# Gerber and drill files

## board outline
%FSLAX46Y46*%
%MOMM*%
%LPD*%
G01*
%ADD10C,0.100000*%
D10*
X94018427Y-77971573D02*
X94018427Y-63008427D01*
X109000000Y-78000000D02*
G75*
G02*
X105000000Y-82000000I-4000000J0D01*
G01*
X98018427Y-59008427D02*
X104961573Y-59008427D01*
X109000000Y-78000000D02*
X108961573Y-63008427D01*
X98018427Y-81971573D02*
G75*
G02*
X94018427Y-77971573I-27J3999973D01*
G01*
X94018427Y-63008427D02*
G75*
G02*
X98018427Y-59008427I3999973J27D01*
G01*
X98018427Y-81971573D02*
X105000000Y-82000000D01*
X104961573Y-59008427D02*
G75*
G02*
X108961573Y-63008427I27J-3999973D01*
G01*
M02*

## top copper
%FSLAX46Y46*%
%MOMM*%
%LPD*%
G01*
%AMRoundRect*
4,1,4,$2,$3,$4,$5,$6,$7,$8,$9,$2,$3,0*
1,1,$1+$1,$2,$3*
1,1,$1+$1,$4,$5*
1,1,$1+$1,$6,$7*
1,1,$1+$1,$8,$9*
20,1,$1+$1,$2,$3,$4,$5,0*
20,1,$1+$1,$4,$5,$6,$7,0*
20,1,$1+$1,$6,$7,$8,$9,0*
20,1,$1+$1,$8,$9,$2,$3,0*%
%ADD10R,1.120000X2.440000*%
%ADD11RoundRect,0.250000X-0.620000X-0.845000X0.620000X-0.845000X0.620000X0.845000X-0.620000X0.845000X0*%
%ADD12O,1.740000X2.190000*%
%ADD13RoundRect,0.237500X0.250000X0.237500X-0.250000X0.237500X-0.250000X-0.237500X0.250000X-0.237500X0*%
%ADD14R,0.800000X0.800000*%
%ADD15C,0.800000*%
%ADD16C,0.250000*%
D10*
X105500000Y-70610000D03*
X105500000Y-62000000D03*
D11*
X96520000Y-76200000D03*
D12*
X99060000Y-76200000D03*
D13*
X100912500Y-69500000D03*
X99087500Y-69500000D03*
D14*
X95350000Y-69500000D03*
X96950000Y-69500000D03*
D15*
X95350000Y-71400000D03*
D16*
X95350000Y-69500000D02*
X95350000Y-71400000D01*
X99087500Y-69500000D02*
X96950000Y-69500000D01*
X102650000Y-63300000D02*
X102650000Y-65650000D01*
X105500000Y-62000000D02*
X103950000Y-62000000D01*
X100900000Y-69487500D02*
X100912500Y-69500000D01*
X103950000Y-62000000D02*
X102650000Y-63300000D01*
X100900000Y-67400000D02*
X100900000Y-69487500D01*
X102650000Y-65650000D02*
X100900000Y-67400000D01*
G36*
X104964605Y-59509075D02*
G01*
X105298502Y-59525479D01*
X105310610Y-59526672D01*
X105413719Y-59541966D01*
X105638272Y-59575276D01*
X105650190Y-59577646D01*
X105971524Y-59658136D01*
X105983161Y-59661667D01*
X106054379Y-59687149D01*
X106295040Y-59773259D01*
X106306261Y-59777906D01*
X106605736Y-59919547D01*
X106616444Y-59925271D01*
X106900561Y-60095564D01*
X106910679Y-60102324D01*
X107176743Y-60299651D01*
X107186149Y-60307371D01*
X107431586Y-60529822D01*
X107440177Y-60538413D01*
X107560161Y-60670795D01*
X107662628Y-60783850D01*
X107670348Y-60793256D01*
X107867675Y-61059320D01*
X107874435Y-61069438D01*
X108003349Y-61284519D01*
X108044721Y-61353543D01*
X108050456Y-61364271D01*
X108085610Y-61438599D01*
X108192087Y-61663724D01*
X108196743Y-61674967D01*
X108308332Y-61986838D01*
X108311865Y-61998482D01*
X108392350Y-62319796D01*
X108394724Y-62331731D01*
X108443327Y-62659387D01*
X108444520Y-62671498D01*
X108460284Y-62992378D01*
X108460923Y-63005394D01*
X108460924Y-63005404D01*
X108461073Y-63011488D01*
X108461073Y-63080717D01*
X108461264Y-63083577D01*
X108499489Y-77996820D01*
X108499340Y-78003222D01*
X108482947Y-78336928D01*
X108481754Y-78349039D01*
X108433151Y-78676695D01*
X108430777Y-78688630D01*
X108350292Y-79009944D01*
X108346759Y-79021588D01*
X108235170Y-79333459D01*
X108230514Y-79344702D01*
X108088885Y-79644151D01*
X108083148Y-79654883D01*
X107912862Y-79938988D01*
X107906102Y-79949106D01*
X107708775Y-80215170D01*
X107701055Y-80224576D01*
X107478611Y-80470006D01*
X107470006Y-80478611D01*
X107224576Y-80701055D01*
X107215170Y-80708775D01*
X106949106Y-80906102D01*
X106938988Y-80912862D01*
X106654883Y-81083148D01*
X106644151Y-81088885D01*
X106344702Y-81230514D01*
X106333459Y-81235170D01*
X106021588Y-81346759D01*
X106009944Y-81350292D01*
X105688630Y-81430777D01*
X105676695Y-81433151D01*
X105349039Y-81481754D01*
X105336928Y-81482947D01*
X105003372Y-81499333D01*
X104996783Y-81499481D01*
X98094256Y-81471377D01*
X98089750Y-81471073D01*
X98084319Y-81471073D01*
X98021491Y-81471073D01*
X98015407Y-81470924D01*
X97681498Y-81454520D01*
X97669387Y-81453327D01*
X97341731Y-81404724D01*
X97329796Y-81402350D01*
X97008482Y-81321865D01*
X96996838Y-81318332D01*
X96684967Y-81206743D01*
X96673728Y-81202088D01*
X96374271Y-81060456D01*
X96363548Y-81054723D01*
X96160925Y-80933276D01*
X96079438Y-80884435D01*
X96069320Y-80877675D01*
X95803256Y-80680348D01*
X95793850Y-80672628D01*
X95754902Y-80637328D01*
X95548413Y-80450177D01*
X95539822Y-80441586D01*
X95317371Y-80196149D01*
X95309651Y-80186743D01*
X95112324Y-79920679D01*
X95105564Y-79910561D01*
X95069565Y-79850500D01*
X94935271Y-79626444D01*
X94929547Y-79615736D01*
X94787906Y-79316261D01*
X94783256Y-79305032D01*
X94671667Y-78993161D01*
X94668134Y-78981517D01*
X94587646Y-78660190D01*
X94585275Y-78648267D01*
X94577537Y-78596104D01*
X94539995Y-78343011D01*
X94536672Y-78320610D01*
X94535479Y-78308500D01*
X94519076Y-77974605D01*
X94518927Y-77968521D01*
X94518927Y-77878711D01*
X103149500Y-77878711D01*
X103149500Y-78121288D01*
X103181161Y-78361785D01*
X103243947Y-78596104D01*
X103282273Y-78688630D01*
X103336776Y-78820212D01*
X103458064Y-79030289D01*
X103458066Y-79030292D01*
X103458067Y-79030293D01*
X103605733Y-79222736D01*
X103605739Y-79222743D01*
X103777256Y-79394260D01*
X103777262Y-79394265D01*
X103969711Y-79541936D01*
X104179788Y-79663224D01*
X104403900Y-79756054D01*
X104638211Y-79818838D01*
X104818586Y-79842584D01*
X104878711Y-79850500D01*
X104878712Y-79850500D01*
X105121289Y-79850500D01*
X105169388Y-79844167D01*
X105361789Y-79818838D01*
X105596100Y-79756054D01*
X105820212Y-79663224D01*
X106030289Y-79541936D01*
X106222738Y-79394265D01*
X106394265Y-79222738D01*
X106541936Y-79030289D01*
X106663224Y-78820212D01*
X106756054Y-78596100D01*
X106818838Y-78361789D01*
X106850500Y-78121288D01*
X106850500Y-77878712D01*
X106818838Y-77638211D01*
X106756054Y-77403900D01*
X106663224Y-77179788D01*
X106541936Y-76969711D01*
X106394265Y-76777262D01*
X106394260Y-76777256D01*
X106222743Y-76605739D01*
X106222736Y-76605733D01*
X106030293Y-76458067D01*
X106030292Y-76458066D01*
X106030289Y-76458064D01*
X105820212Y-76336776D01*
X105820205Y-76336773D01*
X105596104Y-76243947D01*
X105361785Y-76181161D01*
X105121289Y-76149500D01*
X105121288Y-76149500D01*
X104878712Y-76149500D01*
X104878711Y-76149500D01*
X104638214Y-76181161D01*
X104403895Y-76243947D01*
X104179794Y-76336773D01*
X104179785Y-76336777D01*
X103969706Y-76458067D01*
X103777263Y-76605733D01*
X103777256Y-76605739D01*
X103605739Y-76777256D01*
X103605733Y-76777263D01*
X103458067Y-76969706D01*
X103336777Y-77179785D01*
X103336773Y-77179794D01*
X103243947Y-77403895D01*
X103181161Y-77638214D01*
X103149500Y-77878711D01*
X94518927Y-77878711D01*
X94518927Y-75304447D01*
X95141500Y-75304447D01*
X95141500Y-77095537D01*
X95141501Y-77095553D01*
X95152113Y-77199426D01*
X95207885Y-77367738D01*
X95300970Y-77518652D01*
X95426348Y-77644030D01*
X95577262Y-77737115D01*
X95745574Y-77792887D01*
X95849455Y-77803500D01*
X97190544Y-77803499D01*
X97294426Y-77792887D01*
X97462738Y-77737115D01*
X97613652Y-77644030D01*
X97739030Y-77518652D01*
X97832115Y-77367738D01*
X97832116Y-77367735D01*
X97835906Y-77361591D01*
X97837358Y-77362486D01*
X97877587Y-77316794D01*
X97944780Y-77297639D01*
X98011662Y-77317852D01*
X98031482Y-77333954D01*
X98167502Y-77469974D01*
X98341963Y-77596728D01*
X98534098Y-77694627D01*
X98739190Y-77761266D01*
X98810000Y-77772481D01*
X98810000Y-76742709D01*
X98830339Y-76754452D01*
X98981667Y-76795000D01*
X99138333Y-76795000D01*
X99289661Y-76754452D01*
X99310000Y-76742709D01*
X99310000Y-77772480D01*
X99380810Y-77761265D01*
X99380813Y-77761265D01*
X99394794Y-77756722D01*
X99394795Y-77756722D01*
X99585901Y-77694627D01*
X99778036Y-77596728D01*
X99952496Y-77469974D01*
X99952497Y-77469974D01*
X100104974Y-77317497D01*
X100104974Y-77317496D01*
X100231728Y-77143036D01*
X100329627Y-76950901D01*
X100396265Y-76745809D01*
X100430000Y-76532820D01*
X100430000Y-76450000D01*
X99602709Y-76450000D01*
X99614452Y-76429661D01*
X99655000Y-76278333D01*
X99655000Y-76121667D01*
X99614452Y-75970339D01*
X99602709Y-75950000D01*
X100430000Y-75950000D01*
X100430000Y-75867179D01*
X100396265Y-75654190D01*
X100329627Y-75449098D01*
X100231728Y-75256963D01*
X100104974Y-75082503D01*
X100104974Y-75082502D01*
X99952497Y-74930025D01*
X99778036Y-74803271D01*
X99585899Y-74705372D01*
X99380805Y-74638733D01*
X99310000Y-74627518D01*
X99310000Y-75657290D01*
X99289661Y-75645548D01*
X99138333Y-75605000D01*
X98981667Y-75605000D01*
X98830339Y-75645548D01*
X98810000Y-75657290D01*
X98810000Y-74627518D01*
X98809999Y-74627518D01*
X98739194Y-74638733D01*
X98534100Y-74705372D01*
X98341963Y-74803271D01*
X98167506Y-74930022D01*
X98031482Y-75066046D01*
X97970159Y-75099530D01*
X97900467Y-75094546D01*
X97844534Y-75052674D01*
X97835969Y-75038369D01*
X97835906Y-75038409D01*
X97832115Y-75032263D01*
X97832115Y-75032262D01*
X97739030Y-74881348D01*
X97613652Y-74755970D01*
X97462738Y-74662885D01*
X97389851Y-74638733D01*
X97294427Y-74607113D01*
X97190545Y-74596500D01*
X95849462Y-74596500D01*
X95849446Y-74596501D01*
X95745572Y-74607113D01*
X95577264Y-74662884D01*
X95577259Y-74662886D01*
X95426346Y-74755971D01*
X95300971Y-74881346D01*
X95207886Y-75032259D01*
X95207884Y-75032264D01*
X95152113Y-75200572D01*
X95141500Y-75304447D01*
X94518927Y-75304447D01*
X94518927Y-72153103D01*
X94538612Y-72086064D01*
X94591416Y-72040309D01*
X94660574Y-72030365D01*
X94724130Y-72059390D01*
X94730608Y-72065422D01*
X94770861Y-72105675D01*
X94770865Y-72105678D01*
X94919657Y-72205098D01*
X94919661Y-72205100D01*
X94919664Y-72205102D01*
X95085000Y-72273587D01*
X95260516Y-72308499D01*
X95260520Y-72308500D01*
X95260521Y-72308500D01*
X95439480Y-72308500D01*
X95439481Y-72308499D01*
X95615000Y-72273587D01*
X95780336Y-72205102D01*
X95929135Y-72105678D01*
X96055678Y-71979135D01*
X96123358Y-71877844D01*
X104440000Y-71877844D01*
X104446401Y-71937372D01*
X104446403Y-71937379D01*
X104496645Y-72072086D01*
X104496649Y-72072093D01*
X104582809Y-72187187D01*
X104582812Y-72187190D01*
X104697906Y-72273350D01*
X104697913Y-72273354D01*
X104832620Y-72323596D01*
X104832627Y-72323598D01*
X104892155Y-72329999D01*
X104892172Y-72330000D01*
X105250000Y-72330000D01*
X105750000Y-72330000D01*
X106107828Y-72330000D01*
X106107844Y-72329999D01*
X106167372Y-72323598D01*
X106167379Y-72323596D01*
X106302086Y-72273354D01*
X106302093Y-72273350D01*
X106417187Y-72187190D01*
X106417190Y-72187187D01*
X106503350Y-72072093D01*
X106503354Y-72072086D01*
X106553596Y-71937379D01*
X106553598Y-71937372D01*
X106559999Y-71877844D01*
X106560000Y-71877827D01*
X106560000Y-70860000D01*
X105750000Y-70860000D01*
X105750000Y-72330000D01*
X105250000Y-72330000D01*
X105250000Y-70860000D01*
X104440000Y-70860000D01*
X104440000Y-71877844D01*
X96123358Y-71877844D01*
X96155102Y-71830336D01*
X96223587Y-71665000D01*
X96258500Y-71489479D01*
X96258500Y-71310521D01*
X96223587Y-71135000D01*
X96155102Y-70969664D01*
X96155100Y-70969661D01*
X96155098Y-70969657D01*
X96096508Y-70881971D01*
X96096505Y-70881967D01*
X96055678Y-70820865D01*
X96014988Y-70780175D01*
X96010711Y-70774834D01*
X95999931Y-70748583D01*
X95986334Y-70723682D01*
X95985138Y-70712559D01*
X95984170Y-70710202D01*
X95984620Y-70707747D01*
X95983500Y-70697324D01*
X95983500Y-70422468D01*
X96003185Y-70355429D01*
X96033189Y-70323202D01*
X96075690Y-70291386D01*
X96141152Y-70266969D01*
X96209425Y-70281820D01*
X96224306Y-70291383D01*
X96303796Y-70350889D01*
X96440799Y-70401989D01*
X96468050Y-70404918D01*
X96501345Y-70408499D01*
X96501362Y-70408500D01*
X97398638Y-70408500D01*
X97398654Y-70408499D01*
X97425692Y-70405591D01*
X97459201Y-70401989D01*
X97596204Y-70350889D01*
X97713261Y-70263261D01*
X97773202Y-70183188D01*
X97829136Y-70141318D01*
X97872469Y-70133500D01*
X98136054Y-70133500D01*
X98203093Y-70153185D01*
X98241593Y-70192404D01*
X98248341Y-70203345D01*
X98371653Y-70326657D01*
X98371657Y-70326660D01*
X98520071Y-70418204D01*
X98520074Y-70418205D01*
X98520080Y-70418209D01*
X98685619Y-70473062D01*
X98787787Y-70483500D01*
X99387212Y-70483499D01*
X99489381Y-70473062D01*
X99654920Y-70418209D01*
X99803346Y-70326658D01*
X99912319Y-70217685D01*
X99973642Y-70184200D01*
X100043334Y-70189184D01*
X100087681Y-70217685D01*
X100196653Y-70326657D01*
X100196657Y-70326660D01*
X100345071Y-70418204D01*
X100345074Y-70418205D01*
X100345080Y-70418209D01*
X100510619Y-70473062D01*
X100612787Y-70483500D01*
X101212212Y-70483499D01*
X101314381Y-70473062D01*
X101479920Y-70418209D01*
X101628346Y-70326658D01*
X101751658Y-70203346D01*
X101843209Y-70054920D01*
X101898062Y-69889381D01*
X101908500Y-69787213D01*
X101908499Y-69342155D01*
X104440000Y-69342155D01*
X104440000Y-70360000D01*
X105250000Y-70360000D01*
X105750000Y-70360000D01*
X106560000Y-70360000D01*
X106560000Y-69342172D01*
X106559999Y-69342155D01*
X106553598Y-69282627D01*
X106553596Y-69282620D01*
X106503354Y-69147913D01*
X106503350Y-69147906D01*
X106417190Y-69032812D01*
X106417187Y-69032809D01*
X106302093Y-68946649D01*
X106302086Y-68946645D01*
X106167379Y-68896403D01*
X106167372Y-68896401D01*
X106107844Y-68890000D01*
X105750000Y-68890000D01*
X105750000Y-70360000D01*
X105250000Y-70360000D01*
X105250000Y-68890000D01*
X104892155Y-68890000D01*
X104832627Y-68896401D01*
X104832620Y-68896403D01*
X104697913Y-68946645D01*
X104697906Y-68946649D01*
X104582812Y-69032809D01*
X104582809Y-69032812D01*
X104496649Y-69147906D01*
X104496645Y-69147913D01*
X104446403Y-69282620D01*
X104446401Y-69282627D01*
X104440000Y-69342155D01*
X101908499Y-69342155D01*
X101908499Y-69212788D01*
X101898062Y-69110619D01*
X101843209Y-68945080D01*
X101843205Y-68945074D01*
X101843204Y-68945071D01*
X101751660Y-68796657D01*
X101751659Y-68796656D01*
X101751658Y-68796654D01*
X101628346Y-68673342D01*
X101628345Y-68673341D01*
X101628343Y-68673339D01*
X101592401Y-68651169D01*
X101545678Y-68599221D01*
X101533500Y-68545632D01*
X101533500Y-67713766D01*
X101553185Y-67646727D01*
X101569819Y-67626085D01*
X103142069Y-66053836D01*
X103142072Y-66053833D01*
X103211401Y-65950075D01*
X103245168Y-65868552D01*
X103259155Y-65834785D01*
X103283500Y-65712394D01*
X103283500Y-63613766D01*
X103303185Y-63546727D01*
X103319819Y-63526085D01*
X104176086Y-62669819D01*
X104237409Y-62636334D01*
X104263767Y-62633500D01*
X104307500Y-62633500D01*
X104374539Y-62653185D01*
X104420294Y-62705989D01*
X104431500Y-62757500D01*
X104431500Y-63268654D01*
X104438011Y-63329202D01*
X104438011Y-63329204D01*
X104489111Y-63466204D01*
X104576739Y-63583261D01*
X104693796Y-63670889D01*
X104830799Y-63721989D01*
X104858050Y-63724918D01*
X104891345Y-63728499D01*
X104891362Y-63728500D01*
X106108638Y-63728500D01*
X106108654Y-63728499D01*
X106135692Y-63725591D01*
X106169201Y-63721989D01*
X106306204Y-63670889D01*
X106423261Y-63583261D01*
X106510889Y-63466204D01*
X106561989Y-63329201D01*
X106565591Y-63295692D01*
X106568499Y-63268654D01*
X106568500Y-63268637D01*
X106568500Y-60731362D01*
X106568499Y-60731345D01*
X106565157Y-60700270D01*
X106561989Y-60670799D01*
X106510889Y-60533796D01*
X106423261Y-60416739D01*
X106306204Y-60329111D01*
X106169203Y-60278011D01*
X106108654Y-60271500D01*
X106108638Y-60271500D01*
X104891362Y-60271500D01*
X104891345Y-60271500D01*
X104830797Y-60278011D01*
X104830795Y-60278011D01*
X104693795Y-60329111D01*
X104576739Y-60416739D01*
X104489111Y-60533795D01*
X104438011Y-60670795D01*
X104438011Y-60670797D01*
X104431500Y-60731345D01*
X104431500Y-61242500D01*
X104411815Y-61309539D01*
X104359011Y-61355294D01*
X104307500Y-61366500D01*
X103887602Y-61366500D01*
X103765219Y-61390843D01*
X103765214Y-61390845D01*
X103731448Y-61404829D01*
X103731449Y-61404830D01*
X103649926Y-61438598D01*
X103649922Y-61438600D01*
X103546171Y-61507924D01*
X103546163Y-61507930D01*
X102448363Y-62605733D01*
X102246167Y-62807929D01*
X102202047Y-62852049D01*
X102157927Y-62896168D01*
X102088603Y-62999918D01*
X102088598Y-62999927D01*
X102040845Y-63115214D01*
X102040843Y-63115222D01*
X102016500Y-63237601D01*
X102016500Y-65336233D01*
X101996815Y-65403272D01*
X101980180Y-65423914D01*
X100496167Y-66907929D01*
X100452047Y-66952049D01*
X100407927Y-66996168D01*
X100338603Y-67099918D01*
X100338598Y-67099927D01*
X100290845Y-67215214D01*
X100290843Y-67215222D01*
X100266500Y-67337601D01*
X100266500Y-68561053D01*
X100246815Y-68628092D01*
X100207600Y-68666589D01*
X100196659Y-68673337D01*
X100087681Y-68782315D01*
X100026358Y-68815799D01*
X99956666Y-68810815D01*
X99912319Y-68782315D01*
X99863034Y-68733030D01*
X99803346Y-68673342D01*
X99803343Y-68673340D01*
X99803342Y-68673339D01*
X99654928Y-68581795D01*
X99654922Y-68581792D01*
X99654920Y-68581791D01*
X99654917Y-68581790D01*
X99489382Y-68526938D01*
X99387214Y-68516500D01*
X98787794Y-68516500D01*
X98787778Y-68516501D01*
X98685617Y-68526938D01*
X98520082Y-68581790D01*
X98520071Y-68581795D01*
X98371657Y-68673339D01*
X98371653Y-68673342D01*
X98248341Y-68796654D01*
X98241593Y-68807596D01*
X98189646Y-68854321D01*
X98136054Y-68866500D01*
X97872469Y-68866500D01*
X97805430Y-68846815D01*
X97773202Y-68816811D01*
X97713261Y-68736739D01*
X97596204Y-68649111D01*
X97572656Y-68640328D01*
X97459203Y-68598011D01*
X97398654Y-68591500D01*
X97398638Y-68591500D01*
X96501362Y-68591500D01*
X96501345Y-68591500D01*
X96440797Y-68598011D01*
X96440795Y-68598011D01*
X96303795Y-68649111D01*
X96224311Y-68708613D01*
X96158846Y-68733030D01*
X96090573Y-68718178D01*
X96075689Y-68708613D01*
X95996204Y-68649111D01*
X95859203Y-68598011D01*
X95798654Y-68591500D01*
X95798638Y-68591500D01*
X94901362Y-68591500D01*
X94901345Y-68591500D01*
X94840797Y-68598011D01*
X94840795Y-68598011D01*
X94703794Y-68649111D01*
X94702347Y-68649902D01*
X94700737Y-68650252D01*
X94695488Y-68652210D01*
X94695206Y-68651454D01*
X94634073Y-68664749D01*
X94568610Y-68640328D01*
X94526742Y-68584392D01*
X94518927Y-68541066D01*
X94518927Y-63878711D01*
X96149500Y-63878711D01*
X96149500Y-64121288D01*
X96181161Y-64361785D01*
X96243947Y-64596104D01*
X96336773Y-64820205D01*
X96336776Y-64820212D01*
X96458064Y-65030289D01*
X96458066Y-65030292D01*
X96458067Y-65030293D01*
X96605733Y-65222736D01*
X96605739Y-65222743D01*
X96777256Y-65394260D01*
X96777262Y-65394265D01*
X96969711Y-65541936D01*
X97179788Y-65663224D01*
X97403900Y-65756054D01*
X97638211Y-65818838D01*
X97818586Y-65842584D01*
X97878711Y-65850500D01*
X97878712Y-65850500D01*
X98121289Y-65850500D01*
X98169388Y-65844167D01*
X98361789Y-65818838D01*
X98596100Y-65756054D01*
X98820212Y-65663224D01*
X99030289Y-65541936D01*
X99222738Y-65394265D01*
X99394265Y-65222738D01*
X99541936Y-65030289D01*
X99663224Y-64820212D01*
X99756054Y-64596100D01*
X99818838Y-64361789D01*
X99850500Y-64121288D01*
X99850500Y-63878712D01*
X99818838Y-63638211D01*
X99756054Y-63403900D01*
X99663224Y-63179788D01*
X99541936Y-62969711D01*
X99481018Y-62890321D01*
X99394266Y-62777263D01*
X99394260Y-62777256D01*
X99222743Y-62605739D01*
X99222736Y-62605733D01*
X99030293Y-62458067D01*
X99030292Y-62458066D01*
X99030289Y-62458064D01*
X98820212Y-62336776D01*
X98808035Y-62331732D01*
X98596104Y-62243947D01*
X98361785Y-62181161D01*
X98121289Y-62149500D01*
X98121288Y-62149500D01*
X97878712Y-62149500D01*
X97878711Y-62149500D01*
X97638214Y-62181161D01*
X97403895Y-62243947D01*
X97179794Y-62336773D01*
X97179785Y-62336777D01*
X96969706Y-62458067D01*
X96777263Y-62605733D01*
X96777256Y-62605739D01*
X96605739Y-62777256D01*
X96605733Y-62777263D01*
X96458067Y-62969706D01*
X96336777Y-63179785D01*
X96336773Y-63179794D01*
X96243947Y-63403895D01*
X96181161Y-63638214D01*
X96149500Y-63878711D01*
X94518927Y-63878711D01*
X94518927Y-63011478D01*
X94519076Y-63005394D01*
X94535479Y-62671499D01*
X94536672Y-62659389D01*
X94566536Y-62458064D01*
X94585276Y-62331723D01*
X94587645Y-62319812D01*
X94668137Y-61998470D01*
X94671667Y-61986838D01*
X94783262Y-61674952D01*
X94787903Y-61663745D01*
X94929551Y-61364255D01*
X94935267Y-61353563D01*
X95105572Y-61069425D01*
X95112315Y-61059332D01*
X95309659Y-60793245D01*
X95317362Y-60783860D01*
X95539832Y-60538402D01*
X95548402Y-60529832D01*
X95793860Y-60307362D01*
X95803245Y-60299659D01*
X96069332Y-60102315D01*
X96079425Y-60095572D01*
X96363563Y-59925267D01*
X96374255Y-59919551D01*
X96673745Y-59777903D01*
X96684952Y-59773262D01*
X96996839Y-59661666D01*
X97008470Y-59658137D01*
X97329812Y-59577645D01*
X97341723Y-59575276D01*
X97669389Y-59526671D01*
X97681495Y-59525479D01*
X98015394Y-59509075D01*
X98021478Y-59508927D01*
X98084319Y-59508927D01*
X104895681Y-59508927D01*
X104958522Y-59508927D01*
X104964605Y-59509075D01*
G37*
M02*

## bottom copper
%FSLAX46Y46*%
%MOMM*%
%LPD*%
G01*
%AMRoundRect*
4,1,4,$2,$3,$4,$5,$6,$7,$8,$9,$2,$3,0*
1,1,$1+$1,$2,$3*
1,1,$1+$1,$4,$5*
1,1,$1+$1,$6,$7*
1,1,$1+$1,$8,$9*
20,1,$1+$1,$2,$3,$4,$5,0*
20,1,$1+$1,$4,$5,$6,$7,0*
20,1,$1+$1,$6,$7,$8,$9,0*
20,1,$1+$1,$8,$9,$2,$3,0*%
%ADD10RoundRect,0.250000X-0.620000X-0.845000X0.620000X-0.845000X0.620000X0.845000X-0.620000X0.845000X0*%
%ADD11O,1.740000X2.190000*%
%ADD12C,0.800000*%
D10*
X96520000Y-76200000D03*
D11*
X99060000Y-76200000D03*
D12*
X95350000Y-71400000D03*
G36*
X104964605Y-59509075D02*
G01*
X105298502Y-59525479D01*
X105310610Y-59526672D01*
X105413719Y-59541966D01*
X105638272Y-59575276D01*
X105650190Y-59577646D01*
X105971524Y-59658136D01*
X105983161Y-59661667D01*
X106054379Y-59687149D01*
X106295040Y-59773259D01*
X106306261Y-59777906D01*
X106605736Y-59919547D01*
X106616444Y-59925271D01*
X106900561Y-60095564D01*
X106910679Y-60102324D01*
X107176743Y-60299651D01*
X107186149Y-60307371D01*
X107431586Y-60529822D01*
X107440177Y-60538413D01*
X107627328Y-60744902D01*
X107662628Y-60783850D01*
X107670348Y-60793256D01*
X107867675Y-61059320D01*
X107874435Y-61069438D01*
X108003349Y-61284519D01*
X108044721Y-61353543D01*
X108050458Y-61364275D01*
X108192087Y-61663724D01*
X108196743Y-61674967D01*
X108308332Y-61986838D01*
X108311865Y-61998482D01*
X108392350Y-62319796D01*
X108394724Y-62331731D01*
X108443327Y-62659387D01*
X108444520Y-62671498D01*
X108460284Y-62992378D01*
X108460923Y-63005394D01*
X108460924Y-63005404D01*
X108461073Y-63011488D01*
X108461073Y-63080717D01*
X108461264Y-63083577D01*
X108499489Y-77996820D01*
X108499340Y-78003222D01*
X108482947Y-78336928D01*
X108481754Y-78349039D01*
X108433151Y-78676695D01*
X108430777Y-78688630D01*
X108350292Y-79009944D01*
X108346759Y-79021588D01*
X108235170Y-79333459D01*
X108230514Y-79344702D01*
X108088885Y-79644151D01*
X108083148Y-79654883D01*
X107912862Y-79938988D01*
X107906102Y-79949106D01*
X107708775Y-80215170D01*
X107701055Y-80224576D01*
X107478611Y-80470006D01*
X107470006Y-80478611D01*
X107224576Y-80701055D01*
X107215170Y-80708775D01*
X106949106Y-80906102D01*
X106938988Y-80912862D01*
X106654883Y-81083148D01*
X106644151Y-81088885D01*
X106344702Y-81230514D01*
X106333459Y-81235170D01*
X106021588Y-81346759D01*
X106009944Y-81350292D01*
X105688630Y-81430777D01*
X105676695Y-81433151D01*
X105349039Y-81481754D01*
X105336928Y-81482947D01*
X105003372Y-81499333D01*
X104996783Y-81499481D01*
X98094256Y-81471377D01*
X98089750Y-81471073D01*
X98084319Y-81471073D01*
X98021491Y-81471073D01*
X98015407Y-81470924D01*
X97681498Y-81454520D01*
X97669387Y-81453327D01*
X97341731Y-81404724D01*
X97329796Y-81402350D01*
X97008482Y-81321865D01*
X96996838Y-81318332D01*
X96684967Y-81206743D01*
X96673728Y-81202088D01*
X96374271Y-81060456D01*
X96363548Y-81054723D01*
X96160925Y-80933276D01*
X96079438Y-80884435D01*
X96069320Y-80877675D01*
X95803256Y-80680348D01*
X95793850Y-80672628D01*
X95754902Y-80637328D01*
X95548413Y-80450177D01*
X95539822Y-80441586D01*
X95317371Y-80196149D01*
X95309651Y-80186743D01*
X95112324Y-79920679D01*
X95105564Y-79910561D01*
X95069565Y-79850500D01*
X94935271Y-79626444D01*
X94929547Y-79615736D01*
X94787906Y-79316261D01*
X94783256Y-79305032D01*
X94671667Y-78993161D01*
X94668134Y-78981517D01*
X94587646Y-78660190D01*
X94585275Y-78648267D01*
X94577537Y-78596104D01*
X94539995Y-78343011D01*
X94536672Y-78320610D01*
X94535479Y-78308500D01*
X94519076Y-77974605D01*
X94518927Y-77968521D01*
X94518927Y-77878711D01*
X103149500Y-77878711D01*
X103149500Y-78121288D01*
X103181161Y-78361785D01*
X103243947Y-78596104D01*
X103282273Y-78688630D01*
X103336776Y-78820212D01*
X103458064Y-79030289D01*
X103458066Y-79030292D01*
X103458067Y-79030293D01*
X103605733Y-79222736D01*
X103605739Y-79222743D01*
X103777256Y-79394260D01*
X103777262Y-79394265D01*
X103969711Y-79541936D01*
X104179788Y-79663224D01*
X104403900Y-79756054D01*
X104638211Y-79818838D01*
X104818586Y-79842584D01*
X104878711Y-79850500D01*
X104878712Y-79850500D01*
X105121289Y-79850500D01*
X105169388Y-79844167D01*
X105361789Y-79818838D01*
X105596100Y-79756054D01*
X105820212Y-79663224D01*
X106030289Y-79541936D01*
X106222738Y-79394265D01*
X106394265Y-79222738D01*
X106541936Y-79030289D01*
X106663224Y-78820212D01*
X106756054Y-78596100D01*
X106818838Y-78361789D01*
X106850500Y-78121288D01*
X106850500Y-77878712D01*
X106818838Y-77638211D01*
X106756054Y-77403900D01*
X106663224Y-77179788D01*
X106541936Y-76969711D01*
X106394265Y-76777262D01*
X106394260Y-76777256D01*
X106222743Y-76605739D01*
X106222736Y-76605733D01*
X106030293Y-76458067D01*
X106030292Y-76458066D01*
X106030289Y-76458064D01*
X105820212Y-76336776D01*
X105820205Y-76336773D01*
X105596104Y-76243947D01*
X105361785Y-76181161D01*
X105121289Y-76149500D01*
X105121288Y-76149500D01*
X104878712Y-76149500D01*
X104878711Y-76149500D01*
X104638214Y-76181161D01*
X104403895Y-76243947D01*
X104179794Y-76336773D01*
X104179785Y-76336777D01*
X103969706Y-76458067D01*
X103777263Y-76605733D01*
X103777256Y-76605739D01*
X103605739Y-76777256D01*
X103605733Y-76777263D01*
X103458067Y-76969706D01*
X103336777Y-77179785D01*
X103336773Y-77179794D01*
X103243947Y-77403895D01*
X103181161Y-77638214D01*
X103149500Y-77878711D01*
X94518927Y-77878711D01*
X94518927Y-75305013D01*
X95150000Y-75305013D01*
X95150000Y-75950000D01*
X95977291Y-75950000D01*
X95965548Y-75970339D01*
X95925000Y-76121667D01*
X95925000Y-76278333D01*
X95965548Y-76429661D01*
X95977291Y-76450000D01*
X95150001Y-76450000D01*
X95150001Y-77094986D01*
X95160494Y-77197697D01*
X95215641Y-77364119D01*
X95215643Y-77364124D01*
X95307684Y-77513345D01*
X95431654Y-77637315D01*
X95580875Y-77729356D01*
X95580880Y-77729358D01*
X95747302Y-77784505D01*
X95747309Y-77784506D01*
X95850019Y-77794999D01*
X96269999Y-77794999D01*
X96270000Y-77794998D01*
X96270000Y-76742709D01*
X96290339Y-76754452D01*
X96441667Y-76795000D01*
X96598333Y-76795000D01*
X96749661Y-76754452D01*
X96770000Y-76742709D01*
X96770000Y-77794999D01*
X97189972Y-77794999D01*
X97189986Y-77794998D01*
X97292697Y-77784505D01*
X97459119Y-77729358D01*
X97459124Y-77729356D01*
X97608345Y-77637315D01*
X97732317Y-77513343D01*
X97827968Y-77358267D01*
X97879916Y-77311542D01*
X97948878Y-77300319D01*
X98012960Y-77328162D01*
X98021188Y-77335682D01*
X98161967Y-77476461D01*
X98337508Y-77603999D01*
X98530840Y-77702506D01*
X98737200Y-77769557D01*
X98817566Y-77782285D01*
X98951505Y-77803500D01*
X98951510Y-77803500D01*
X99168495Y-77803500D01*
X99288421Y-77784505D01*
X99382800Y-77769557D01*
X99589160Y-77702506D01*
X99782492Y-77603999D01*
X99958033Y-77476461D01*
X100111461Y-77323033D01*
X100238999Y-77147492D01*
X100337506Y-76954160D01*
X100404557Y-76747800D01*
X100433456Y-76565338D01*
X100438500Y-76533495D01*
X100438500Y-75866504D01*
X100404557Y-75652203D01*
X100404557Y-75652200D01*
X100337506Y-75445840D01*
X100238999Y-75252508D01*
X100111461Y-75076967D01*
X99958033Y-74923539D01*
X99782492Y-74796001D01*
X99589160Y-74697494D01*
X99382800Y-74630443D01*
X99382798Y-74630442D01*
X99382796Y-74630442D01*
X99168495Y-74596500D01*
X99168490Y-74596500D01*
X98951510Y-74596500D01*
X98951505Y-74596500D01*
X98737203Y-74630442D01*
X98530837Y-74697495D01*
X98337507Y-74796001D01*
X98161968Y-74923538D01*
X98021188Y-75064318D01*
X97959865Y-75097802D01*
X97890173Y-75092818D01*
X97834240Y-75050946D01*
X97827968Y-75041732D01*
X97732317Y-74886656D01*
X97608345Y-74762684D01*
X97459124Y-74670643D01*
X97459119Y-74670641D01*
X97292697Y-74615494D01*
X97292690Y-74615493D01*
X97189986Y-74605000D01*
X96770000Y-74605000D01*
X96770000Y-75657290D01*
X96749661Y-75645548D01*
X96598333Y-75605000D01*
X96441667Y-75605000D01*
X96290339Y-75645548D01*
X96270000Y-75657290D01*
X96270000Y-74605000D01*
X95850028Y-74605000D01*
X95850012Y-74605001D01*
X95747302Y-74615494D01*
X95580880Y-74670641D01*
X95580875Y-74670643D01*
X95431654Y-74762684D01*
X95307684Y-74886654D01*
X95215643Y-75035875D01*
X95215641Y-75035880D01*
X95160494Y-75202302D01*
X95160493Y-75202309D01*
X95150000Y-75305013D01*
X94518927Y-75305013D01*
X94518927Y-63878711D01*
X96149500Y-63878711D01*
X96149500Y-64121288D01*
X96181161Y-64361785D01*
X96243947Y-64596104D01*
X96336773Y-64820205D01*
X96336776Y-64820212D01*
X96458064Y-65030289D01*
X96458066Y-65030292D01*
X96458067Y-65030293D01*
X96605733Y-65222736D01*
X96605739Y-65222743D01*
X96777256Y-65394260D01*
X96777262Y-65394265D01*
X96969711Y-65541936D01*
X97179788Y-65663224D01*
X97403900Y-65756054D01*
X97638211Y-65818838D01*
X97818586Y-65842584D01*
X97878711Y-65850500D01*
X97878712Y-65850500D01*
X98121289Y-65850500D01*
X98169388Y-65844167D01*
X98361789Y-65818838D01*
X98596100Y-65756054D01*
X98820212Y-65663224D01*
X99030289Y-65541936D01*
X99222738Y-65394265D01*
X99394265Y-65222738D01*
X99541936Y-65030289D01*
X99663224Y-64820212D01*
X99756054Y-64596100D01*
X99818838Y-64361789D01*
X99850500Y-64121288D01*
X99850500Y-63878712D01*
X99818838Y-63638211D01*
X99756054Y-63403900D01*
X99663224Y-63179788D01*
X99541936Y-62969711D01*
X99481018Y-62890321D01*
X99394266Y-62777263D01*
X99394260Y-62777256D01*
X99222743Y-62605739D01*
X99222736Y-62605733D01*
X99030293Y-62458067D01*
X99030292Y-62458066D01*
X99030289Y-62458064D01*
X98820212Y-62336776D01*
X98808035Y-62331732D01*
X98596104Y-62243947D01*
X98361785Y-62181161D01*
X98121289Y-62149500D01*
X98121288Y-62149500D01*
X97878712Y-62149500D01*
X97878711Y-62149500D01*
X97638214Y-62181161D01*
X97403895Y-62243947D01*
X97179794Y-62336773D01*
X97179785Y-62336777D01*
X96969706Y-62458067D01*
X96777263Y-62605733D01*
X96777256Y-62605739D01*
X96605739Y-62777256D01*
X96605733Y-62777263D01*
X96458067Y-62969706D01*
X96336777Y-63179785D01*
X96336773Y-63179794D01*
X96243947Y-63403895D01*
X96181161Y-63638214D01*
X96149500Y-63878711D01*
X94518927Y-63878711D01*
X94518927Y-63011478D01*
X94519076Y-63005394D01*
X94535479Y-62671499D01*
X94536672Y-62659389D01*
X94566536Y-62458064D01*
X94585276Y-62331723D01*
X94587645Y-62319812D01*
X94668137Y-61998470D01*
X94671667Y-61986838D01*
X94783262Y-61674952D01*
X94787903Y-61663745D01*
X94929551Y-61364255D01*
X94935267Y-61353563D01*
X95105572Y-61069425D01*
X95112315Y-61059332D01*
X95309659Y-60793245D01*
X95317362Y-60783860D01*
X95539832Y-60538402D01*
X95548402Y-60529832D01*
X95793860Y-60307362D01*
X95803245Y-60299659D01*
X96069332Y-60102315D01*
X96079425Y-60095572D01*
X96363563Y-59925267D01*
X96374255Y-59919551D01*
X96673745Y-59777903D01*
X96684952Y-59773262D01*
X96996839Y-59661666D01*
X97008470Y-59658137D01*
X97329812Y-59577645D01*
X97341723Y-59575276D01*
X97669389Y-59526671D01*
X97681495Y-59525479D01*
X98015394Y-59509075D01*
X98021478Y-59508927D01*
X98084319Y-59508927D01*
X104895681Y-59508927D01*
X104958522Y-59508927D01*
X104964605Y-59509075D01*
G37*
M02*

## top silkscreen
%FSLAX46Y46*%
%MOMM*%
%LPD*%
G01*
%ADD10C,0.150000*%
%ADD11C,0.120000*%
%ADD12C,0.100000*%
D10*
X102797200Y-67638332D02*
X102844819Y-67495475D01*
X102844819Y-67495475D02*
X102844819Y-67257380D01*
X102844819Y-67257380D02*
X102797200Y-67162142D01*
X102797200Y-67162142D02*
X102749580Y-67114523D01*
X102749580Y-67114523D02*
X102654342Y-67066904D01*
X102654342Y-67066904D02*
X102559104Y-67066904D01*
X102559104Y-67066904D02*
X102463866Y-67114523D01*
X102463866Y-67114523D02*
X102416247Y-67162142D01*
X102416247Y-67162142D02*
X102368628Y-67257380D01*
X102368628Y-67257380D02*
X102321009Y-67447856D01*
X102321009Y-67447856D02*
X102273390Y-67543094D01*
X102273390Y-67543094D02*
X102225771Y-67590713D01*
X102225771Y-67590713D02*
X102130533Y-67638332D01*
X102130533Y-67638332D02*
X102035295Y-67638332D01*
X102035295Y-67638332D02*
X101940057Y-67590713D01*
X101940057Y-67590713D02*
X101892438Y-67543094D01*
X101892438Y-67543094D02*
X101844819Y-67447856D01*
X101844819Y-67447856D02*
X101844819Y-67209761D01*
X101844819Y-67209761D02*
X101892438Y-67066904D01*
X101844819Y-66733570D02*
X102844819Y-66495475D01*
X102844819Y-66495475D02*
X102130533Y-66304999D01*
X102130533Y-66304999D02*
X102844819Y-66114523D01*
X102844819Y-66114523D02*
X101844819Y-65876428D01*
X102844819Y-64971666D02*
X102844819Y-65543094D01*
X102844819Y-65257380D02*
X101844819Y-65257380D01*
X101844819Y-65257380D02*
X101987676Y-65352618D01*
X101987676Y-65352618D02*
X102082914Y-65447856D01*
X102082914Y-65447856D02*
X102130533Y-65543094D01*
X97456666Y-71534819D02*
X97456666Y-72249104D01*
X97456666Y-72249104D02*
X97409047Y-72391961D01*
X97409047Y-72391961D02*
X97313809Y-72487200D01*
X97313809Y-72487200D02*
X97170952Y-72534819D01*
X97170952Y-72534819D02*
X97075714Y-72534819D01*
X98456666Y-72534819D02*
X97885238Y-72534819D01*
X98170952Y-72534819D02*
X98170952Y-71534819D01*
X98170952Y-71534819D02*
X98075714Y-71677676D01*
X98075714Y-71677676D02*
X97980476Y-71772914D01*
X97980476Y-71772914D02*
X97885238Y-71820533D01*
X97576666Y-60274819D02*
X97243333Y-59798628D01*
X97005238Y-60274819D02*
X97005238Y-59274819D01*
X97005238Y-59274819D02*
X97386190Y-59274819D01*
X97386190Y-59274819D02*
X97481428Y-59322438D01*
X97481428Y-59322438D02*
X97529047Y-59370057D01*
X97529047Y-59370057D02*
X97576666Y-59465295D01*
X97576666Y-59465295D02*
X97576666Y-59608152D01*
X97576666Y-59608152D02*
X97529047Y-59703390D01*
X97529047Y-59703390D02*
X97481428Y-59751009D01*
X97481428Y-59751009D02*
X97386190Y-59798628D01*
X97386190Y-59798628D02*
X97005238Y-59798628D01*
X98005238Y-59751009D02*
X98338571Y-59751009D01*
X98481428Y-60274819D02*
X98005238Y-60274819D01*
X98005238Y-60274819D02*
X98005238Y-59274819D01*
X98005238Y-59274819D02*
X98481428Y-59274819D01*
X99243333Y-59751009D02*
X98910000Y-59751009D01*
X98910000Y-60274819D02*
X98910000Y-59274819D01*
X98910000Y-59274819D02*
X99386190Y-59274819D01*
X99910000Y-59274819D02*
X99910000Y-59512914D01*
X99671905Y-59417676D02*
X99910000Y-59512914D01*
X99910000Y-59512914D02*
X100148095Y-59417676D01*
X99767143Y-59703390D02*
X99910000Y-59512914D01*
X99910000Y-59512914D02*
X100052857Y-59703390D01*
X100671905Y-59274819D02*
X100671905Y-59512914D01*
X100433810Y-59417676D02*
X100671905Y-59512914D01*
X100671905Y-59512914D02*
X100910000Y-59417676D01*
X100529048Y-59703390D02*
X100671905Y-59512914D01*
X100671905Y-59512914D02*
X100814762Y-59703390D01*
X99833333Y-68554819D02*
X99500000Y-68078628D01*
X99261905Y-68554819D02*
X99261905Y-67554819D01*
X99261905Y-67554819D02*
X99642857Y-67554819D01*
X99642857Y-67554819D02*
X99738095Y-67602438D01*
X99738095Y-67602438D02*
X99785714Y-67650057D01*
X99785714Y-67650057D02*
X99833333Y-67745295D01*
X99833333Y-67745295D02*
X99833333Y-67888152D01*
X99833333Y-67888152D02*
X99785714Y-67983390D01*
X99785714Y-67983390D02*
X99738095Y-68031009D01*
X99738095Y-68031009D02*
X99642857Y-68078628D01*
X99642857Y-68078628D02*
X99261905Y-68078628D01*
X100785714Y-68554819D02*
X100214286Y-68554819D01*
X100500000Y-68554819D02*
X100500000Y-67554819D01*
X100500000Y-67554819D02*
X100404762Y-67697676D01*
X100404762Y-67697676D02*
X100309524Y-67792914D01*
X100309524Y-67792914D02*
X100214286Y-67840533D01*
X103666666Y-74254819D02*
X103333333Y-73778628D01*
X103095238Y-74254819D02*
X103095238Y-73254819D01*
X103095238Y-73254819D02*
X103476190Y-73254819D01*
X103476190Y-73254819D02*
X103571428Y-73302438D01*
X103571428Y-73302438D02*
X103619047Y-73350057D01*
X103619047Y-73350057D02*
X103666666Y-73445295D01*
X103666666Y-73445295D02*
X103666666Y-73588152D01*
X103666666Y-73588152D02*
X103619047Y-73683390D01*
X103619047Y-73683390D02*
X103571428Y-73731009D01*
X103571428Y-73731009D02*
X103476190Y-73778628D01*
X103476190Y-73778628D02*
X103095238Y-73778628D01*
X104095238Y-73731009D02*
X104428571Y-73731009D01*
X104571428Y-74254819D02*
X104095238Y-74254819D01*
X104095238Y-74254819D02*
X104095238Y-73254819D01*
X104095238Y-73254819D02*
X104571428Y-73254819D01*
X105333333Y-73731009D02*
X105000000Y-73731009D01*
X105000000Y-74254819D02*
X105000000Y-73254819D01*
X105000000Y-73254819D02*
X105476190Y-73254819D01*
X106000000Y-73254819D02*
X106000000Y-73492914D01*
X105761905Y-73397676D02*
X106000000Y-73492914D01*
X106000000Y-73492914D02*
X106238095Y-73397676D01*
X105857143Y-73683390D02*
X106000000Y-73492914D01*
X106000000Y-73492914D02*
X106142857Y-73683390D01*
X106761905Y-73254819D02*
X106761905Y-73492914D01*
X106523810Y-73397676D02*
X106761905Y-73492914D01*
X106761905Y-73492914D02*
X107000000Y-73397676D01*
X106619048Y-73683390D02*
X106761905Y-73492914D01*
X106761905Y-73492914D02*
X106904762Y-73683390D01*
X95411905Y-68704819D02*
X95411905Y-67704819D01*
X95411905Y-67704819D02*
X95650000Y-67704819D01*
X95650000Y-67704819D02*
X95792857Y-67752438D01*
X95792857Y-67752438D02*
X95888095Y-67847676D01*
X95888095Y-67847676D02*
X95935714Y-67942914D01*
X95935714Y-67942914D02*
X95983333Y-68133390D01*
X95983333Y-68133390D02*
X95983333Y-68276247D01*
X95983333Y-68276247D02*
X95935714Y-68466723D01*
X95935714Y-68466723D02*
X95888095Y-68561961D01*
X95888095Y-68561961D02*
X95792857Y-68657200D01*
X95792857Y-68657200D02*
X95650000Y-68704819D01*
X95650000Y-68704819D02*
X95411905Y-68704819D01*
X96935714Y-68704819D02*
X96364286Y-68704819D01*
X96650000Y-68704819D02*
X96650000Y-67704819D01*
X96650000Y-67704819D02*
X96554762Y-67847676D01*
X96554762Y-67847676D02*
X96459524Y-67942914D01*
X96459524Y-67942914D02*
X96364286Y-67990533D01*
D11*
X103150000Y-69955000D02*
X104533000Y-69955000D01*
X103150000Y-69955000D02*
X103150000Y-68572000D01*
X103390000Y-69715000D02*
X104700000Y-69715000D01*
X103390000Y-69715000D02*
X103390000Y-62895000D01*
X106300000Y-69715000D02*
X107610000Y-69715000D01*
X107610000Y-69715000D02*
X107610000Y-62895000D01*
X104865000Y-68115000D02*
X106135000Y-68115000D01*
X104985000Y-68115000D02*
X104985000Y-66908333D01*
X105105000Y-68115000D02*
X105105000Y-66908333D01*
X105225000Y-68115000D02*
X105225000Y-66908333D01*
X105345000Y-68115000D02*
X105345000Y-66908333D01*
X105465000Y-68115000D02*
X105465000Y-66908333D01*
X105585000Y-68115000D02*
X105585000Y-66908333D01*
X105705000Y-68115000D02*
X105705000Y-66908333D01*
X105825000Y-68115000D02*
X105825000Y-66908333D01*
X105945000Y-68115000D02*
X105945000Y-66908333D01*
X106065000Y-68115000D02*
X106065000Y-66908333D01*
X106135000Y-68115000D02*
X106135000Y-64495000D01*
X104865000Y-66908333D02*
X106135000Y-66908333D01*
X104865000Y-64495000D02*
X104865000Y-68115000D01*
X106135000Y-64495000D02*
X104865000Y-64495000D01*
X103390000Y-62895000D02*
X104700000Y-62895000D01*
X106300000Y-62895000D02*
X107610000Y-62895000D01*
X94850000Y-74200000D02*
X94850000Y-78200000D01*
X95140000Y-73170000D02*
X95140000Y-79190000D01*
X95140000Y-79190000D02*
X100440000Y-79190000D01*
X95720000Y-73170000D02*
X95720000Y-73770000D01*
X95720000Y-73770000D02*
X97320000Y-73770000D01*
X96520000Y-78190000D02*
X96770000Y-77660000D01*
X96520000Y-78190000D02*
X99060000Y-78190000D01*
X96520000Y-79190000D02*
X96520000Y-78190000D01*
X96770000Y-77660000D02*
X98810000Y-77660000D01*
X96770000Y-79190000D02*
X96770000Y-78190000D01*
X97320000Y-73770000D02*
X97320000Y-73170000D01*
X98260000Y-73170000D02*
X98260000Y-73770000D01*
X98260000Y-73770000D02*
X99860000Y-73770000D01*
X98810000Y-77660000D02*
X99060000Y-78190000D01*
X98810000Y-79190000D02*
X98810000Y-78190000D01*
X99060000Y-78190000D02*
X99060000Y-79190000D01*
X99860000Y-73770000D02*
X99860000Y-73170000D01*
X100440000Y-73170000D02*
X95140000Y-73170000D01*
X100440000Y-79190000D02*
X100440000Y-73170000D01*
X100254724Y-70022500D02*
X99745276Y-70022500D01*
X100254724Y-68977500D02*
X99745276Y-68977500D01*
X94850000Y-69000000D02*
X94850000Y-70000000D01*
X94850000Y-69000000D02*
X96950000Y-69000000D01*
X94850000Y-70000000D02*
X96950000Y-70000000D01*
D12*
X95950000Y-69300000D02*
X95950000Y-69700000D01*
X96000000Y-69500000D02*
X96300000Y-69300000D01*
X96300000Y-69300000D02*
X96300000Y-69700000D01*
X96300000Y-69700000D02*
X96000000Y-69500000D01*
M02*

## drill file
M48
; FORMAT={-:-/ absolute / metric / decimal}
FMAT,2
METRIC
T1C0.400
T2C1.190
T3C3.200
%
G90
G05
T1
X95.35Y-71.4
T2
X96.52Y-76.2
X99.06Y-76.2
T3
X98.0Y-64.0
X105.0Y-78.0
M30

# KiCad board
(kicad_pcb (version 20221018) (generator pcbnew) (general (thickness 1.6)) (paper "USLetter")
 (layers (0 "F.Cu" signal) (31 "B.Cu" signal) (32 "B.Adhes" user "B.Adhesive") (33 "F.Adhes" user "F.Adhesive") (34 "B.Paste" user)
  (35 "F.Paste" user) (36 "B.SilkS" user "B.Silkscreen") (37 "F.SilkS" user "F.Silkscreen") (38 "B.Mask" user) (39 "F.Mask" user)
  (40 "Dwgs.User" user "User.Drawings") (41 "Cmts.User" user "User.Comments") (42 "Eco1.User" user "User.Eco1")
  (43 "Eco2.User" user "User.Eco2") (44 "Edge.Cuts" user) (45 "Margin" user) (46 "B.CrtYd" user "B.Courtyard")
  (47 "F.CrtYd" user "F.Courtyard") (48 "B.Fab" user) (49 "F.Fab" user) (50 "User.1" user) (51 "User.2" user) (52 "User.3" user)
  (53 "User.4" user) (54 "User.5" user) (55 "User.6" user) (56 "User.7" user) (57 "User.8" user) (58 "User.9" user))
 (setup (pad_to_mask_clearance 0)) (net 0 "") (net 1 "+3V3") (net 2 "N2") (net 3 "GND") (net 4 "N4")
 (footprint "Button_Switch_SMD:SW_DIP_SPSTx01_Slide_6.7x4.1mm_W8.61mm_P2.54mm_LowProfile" (layer "F.Cu") (at 105.5 66.305 90)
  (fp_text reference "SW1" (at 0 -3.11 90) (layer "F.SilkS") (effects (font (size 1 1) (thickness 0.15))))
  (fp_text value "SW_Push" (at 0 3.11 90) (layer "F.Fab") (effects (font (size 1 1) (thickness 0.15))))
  (fp_line (start -3.65 -2.35) (end -3.65 -0.967) (stroke (width 0.12) (type solid)) (layer "F.SilkS"))
  (fp_line (start -3.65 -2.35) (end -2.267 -2.35) (stroke (width 0.12) (type solid)) (layer "F.SilkS"))
  (fp_line (start -3.41 -2.11) (end -3.41 -0.8) (stroke (width 0.12) (type solid)) (layer "F.SilkS"))
  (fp_line (start -3.41 -2.11) (end 3.41 -2.11) (stroke (width 0.12) (type solid)) (layer "F.SilkS"))
  (fp_line (start -3.41 0.8) (end -3.41 2.11) (stroke (width 0.12) (type solid)) (layer "F.SilkS"))
  (fp_line (start -3.41 2.11) (end 3.41 2.11) (stroke (width 0.12) (type solid)) (layer "F.SilkS"))
  (fp_line (start -1.81 -0.635) (end -1.81 0.635) (stroke (width 0.12) (type solid)) (layer "F.SilkS"))
  (fp_line (start -1.81 -0.515) (end -0.603333 -0.515) (stroke (width 0.12) (type solid)) (layer "F.SilkS"))
  (fp_line (start -1.81 -0.395) (end -0.603333 -0.395) (stroke (width 0.12) (type solid)) (layer "F.SilkS"))
  (fp_line (start -1.81 -0.275) (end -0.603333 -0.275) (stroke (width 0.12) (type solid)) (layer "F.SilkS"))
  (fp_line (start -1.81 -0.155) (end -0.603333 -0.155) (stroke (width 0.12) (type solid)) (layer "F.SilkS"))
  (fp_line (start -1.81 -0.035) (end -0.603333 -0.035) (stroke (width 0.12) (type solid)) (layer "F.SilkS"))
  (fp_line (start -1.81 0.085) (end -0.603333 0.085) (stroke (width 0.12) (type solid)) (layer "F.SilkS"))
  (fp_line (start -1.81 0.205) (end -0.603333 0.205) (stroke (width 0.12) (type solid)) (layer "F.SilkS"))
  (fp_line (start -1.81 0.325) (end -0.603333 0.325) (stroke (width 0.12) (type solid)) (layer "F.SilkS"))
  (fp_line (start -1.81 0.445) (end -0.603333 0.445) (stroke (width 0.12) (type solid)) (layer "F.SilkS"))
  (fp_line (start -1.81 0.565) (end -0.603333 0.565) (stroke (width 0.12) (type solid)) (layer "F.SilkS"))
  (fp_line (start -1.81 0.635) (end 1.81 0.635) (stroke (width 0.12) (type solid)) (layer "F.SilkS"))
  (fp_line (start -0.603333 -0.635) (end -0.603333 0.635) (stroke (width 0.12) (type solid)) (layer "F.SilkS"))
  (fp_line (start 1.81 -0.635) (end -1.81 -0.635) (stroke (width 0.12) (type solid)) (layer "F.SilkS"))
  (fp_line (start 1.81 0.635) (end 1.81 -0.635) (stroke (width 0.12) (type solid)) (layer "F.SilkS"))
  (fp_line (start 3.41 -2.11) (end 3.41 -0.8) (stroke (width 0.12) (type solid)) (layer "F.SilkS"))
  (fp_line (start 3.41 0.8) (end 3.41 2.11) (stroke (width 0.12) (type solid)) (layer "F.SilkS"))
  (pad "1" smd rect (at -4.305 0 90) (size 2.44 1.12) (layers "F.Cu" "F.Paste" "F.Mask") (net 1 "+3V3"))
  (pad "2" smd rect (at 4.305 0 90) (size 2.44 1.12) (layers "F.Cu" "F.Paste" "F.Mask") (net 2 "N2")))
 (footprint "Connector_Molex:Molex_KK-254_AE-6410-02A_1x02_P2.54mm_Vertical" (layer "F.Cu") (at 96.52 76.2)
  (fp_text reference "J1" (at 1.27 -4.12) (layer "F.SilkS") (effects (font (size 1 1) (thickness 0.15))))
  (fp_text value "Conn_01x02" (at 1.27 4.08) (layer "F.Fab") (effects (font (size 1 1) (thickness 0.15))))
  (fp_line (start -1.67 -2) (end -1.67 2) (stroke (width 0.12) (type solid)) (layer "F.SilkS"))
  (fp_line (start -1.38 -3.03) (end -1.38 2.99) (stroke (width 0.12) (type solid)) (layer "F.SilkS"))
  (fp_line (start -1.38 2.99) (end 3.92 2.99) (stroke (width 0.12) (type solid)) (layer "F.SilkS"))
  (fp_line (start -0.8 -3.03) (end -0.8 -2.43) (stroke (width 0.12) (type solid)) (layer "F.SilkS"))
  (fp_line (start -0.8 -2.43) (end 0.8 -2.43) (stroke (width 0.12) (type solid)) (layer "F.SilkS"))
  (fp_line (start 0 1.99) (end 0.25 1.46) (stroke (width 0.12) (type solid)) (layer "F.SilkS"))
  (fp_line (start 0 1.99) (end 2.54 1.99) (stroke (width 0.12) (type solid)) (layer "F.SilkS"))
  (fp_line (start 0 2.99) (end 0 1.99) (stroke (width 0.12) (type solid)) (layer "F.SilkS"))
  (fp_line (start 0.25 1.46) (end 2.29 1.46) (stroke (width 0.12) (type solid)) (layer "F.SilkS"))
  (fp_line (start 0.25 2.99) (end 0.25 1.99) (stroke (width 0.12) (type solid)) (layer "F.SilkS"))
  (fp_line (start 0.8 -2.43) (end 0.8 -3.03) (stroke (width 0.12) (type solid)) (layer "F.SilkS"))
  (fp_line (start 1.74 -3.03) (end 1.74 -2.43) (stroke (width 0.12) (type solid)) (layer "F.SilkS"))
  (fp_line (start 1.74 -2.43) (end 3.34 -2.43) (stroke (width 0.12) (type solid)) (layer "F.SilkS"))
  (fp_line (start 2.29 1.46) (end 2.54 1.99) (stroke (width 0.12) (type solid)) (layer "F.SilkS"))
  (fp_line (start 2.29 2.99) (end 2.29 1.99) (stroke (width 0.12) (type solid)) (layer "F.SilkS"))
  (fp_line (start 2.54 1.99) (end 2.54 2.99) (stroke (width 0.12) (type solid)) (layer "F.SilkS"))
  (fp_line (start 3.34 -2.43) (end 3.34 -3.03) (stroke (width 0.12) (type solid)) (layer "F.SilkS"))
  (fp_line (start 3.92 -3.03) (end -1.38 -3.03) (stroke (width 0.12) (type solid)) (layer "F.SilkS"))
  (fp_line (start 3.92 2.99) (end 3.92 -3.03) (stroke (width 0.12) (type solid)) (layer "F.SilkS"))
  (pad "1" thru_hole roundrect (at 0 0) (size 1.74 2.19) (drill 1.19) (layers "*.Cu" "*.Mask") (roundrect_rratio 0.143678) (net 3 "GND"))
  (pad "2" thru_hole oval (at 2.54 0) (size 1.74 2.19) (drill 1.19) (layers "*.Cu" "*.Mask") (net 1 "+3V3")))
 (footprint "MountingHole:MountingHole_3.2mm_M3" (layer "F.Cu") (at 98 64)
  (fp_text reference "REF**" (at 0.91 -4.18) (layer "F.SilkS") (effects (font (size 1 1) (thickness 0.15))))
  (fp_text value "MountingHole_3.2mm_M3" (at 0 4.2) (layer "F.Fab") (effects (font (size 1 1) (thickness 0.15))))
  (pad "" np_thru_hole circle (at 0 0) (size 3.2 3.2) (drill 3.2) (layers "*.Cu" "*.Mask")))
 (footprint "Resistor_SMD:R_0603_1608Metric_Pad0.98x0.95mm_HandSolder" (layer "F.Cu") (at 100 69.5 180)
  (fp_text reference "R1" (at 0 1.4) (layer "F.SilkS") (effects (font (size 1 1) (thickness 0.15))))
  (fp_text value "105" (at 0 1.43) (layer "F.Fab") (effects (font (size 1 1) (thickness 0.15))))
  (fp_line (start -0.254724 -0.5225) (end 0.254724 -0.5225) (stroke (width 0.12) (type solid)) (layer "F.SilkS"))
  (fp_line (start -0.254724 0.5225) (end 0.254724 0.5225) (stroke (width 0.12) (type solid)) (layer "F.SilkS"))
  (pad "1" smd roundrect (at -0.9125 0 180) (size 0.975 0.95) (layers "F.Cu" "F.Paste" "F.Mask") (roundrect_rratio 0.25) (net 2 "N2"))
  (pad "2" smd roundrect (at 0.9125 0 180) (size 0.975 0.95) (layers "F.Cu" "F.Paste" "F.Mask") (roundrect_rratio 0.25) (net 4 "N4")))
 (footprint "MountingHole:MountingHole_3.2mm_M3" (layer "F.Cu") (at 105 78)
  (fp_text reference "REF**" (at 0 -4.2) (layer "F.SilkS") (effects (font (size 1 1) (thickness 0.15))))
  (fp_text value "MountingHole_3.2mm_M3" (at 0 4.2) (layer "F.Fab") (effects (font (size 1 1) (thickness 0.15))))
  (pad "" np_thru_hole circle (at 0 0) (size 3.2 3.2) (drill 3.2) (layers "*.Cu" "*.Mask")))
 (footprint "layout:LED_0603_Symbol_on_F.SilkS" (layer "F.Cu") (at 96.15 69.5)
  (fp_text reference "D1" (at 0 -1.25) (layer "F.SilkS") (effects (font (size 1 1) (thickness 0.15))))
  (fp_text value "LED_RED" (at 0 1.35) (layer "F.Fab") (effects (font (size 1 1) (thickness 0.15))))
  (fp_line (start -1.3 -0.5) (end -1.3 0.5) (stroke (width 0.12) (type solid)) (layer "F.SilkS"))
  (fp_line (start -1.3 -0.5) (end 0.8 -0.5) (stroke (width 0.12) (type solid)) (layer "F.SilkS"))
  (fp_line (start -1.3 0.5) (end 0.8 0.5) (stroke (width 0.12) (type solid)) (layer "F.SilkS"))
  (fp_line (start -0.2 -0.2) (end -0.2 0.2) (stroke (width 0.1) (type solid)) (layer "F.SilkS"))
  (fp_line (start -0.15 0) (end 0.15 -0.2) (stroke (width 0.1) (type solid)) (layer "F.SilkS"))
  (fp_line (start 0.15 -0.2) (end 0.15 0.2) (stroke (width 0.1) (type solid)) (layer "F.SilkS"))
  (fp_line (start 0.15 0.2) (end -0.15 0) (stroke (width 0.1) (type solid)) (layer "F.SilkS"))
  (pad "1" smd rect (at -0.8 0 180) (size 0.8 0.8) (layers "F.Cu" "F.Paste" "F.Mask") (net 3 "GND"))
  (pad "2" smd rect (at 0.8 0 180) (size 0.8 0.8) (layers "F.Cu" "F.Paste" "F.Mask") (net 4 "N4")))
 (gr_line (start 94.018427 77.971573) (end 94.018427 63.008427) (stroke (width 0.1) (type default)) (layer "Edge.Cuts"))
 (gr_arc (start 109 78) (mid 107.828427 80.828427) (end 105 82) (stroke (width 0.1) (type default)) (layer "Edge.Cuts"))
 (gr_line (start 98.018427 59.008427) (end 104.961573 59.008427) (stroke (width 0.1) (type default)) (layer "Edge.Cuts"))
 (gr_line (start 109 78) (end 108.961573 63.008427) (stroke (width 0.1) (type default)) (layer "Edge.Cuts"))
 (gr_arc (start 98.018427 81.971573) (mid 95.19 80.8) (end 94.018427 77.971573) (stroke (width 0.1) (type default)) (layer "Edge.Cuts"))
 (gr_arc (start 94.018427 63.008427) (mid 95.19 60.18) (end 98.018427 59.008427) (stroke (width 0.1) (type default)) (layer "Edge.Cuts"))
 (gr_line (start 98.018427 81.971573) (end 105 82) (stroke (width 0.1) (type default)) (layer "Edge.Cuts"))
 (gr_arc (start 104.961573 59.008427) (mid 107.79 60.18) (end 108.961573 63.008427) (stroke (width 0.1) (type default)) (layer "Edge.Cuts"))
 (segment (start 95.35 69.5) (end 95.35 71.4) (width 0.25) (layer "F.Cu") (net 3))
 (via (at 95.35 71.4) (size 0.8) (drill 0.4) (layers "F.Cu" "B.Cu") (free) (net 3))
 (segment (start 99.0875 69.5) (end 96.95 69.5) (width 0.25) (layer "F.Cu") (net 4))
 (segment (start 102.65 63.3) (end 102.65 65.65) (width 0.25) (layer "F.Cu") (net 2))
 (segment (start 105.5 62) (end 103.95 62) (width 0.25) (layer "F.Cu") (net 2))
 (segment (start 100.9 69.4875) (end 100.9125 69.5) (width 0.25) (layer "F.Cu") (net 2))
 (segment (start 103.95 62) (end 102.65 63.3) (width 0.25) (layer "F.Cu") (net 2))
 (segment (start 100.9 67.4) (end 100.9 69.4875) (width 0.25) (layer "F.Cu") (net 2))
 (segment (start 102.65 65.65) (end 100.9 67.4) (width 0.25) (layer "F.Cu") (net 2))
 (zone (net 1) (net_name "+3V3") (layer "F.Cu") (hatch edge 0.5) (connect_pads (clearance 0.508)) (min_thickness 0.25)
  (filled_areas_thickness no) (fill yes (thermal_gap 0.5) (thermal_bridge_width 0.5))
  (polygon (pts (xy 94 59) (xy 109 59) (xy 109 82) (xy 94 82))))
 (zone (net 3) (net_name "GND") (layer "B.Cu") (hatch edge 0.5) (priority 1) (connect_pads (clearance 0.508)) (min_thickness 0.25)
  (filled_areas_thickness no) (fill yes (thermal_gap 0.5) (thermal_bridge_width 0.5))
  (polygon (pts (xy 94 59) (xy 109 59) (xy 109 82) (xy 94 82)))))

